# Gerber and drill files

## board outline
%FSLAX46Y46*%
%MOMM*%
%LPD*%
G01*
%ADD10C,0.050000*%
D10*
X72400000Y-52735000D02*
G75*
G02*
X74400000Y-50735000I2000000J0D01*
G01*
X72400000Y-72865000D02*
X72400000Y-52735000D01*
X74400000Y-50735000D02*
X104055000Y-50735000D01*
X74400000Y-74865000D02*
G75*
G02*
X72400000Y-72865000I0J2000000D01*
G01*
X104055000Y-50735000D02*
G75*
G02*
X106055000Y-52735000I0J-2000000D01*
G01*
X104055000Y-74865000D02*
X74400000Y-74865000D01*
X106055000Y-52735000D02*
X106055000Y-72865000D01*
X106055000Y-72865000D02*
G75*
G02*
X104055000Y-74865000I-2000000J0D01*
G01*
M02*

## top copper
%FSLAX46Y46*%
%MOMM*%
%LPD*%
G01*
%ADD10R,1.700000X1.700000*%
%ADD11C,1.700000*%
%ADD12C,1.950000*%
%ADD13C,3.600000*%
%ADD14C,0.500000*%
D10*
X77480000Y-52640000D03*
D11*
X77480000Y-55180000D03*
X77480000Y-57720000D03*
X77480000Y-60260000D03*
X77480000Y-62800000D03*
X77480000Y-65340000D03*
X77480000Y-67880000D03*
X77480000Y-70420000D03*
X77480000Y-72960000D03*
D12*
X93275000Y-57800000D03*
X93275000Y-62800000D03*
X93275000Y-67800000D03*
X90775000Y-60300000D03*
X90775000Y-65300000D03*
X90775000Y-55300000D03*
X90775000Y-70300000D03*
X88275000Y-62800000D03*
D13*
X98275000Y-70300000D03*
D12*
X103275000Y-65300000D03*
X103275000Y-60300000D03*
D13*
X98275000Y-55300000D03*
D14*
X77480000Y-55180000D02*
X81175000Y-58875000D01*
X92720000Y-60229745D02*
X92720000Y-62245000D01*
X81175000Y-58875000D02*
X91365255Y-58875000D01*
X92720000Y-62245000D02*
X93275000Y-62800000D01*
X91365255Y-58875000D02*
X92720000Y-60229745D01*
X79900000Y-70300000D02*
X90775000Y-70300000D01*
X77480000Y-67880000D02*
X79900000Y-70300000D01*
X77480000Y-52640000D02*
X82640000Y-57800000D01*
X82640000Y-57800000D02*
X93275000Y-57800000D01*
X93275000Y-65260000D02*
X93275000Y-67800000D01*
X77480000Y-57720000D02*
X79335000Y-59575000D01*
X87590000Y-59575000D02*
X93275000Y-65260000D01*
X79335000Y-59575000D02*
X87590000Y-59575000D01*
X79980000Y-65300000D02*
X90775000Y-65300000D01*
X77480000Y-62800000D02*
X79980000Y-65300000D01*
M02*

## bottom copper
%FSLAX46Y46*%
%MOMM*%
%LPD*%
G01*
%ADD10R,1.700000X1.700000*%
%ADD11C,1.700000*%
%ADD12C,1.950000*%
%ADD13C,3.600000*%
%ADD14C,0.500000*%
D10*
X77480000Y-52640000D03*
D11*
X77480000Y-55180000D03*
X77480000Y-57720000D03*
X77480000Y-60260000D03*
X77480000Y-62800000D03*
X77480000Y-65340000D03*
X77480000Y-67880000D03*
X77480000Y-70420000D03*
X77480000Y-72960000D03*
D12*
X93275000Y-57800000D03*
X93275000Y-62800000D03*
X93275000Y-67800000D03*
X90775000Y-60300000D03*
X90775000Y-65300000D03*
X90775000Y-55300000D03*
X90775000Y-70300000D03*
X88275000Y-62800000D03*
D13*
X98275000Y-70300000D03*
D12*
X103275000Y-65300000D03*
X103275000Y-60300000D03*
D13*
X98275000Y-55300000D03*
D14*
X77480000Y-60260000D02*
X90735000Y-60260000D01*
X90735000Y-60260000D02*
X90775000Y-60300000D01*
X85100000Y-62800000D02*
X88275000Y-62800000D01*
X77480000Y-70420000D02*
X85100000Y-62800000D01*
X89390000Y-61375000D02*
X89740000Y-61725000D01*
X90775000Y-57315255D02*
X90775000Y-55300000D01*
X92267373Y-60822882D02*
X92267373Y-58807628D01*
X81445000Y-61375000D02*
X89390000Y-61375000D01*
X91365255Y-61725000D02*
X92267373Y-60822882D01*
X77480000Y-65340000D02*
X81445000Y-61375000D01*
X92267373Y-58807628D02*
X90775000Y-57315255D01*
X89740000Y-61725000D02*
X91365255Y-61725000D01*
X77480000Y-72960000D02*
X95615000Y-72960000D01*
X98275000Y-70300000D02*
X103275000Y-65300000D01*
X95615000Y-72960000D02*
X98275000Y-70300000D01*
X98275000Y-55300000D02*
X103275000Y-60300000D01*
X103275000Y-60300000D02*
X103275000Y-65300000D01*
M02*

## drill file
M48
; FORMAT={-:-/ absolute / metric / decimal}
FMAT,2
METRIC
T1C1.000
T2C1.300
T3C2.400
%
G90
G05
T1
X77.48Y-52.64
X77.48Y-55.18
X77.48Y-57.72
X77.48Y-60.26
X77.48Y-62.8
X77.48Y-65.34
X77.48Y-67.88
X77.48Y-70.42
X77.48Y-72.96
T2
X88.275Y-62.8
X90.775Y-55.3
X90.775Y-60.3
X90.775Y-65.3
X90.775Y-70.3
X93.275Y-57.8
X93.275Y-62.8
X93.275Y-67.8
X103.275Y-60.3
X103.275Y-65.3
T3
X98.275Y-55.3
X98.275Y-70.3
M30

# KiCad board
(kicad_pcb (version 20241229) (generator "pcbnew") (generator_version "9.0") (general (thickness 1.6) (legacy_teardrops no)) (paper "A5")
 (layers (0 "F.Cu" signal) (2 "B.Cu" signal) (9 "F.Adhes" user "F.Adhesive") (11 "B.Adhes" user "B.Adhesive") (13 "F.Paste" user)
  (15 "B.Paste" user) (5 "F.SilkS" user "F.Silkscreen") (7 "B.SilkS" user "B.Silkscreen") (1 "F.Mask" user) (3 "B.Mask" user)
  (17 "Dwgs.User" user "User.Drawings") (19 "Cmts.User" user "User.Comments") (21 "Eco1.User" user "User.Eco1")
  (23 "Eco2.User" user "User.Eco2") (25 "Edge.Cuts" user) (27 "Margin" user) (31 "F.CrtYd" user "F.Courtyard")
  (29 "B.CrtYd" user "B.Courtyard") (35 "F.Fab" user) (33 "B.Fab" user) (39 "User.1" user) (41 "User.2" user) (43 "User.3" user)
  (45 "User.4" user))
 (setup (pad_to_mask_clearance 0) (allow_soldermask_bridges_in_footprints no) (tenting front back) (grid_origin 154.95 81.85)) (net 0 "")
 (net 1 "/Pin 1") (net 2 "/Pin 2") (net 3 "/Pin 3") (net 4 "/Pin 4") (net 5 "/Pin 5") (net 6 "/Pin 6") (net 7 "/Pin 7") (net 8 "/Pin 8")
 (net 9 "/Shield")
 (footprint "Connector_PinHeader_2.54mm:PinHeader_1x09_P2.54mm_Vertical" (layer "F.Cu") (at 77.48 52.64)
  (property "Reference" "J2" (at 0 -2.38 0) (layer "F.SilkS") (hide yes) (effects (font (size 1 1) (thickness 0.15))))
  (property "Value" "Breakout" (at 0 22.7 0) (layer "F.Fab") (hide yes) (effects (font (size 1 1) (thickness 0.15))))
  (pad "1" thru_hole rect (at 0 0) (size 1.7 1.7) (drill 1) (layers "*.Cu" "*.Mask") (remove_unused_layers no) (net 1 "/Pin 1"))
  (pad "2" thru_hole circle (at 0 2.54) (size 1.7 1.7) (drill 1) (layers "*.Cu" "*.Mask") (remove_unused_layers no) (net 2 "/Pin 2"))
  (pad "3" thru_hole circle (at 0 5.08) (size 1.7 1.7) (drill 1) (layers "*.Cu" "*.Mask") (remove_unused_layers no) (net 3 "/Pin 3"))
  (pad "4" thru_hole circle (at 0 7.62) (size 1.7 1.7) (drill 1) (layers "*.Cu" "*.Mask") (remove_unused_layers no) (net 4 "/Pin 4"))
  (pad "5" thru_hole circle (at 0 10.16) (size 1.7 1.7) (drill 1) (layers "*.Cu" "*.Mask") (remove_unused_layers no) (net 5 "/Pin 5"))
  (pad "6" thru_hole circle (at 0 12.7) (size 1.7 1.7) (drill 1) (layers "*.Cu" "*.Mask") (remove_unused_layers no) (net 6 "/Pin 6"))
  (pad "7" thru_hole circle (at 0 15.24) (size 1.7 1.7) (drill 1) (layers "*.Cu" "*.Mask") (remove_unused_layers no) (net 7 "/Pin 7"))
  (pad "8" thru_hole circle (at 0 17.78) (size 1.7 1.7) (drill 1) (layers "*.Cu" "*.Mask") (remove_unused_layers no) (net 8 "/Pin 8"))
  (pad "SH" thru_hole circle (at 0 20.32) (size 1.7 1.7) (drill 1) (layers "*.Cu" "*.Mask") (remove_unused_layers no) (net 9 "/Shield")))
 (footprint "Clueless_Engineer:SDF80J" (layer "F.Cu") (at 93.275 57.8 90)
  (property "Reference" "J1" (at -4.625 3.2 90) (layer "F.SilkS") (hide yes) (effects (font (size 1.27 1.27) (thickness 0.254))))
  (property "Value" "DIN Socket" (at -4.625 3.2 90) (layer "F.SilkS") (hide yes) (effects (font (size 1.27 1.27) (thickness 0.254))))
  (pad "1" thru_hole circle (at 0 0 90) (size 1.95 1.95) (drill 1.3) (layers "*.Cu" "*.Mask") (remove_unused_layers no) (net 1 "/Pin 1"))
  (pad "2" thru_hole circle (at -5 0 90) (size 1.95 1.95) (drill 1.3) (layers "*.Cu" "*.Mask") (remove_unused_layers no) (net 2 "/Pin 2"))
  (pad "3" thru_hole circle (at -10 0 90) (size 1.95 1.95) (drill 1.3) (layers "*.Cu" "*.Mask") (remove_unused_layers no) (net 3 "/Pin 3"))
  (pad "4" thru_hole circle (at -2.5 -2.5 90) (size 1.95 1.95) (drill 1.3) (layers "*.Cu" "*.Mask") (remove_unused_layers no)
   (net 4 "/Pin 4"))
  (pad "5" thru_hole circle (at -7.5 -2.5 90) (size 1.95 1.95) (drill 1.3) (layers "*.Cu" "*.Mask") (remove_unused_layers no)
   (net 5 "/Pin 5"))
  (pad "6" thru_hole circle (at 2.5 -2.5 90) (size 1.95 1.95) (drill 1.3) (layers "*.Cu" "*.Mask") (remove_unused_layers no)
   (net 6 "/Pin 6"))
  (pad "7" thru_hole circle (at -12.5 -2.5 90) (size 1.95 1.95) (drill 1.3) (layers "*.Cu" "*.Mask") (remove_unused_layers no)
   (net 7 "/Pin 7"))
  (pad "8" thru_hole circle (at -5 -5 90) (size 1.95 1.95) (drill 1.3) (layers "*.Cu" "*.Mask") (remove_unused_layers no) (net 8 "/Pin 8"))
  (pad "SH" thru_hole circle (at -12.5 5 90) (size 3.6 3.6) (drill 2.4) (layers "*.Cu" "*.Mask") (remove_unused_layers no) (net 9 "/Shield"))
  (pad "SH" thru_hole circle (at -7.5 10 90) (size 1.95 1.95) (drill 1.3) (layers "*.Cu" "*.Mask") (remove_unused_layers no)
   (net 9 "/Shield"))
  (pad "SH" thru_hole circle (at -2.5 10 90) (size 1.95 1.95) (drill 1.3) (layers "*.Cu" "*.Mask") (remove_unused_layers no)
   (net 9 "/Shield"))
  (pad "SH" thru_hole circle (at 2.5 5 90) (size 3.6 3.6) (drill 2.4) (layers "*.Cu" "*.Mask") (remove_unused_layers no) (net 9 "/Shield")))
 (gr_arc (start 72.4 52.735) (mid 72.985786 51.320786) (end 74.4 50.735) (stroke (width 0.05) (type default)) (layer "Edge.Cuts"))
 (gr_line (start 72.4 72.865) (end 72.4 52.735) (stroke (width 0.05) (type default)) (layer "Edge.Cuts"))
 (gr_line (start 74.4 50.735) (end 104.055 50.735) (stroke (width 0.05) (type default)) (layer "Edge.Cuts"))
 (gr_arc (start 74.4 74.865) (mid 72.985786 74.279214) (end 72.4 72.865) (stroke (width 0.05) (type default)) (layer "Edge.Cuts"))
 (gr_arc (start 104.055 50.735) (mid 105.469214 51.320786) (end 106.055 52.735) (stroke (width 0.05) (type default)) (layer "Edge.Cuts"))
 (gr_line (start 104.055 74.865) (end 74.4 74.865) (stroke (width 0.05) (type default)) (layer "Edge.Cuts"))
 (gr_line (start 106.055 52.735) (end 106.055 72.865) (stroke (width 0.05) (type default)) (layer "Edge.Cuts"))
 (gr_arc (start 106.055 72.865) (mid 105.469214 74.279214) (end 104.055 74.865) (stroke (width 0.05) (type default)) (layer "Edge.Cuts"))
 (segment (start 77.48 60.26) (end 90.735 60.26) (width 0.5) (layer "B.Cu") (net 4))
 (segment (start 90.735 60.26) (end 90.775 60.3) (width 0.5) (layer "B.Cu") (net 4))
 (segment (start 85.1 62.8) (end 88.275 62.8) (width 0.5) (layer "B.Cu") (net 8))
 (segment (start 77.48 70.42) (end 85.1 62.8) (width 0.5) (layer "B.Cu") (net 8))
 (segment (start 77.48 55.18) (end 81.175 58.875) (width 0.5) (layer "F.Cu") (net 2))
 (segment (start 92.72 60.229745) (end 92.72 62.245) (width 0.5) (layer "F.Cu") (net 2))
 (segment (start 81.175 58.875) (end 91.365255 58.875) (width 0.5) (layer "F.Cu") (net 2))
 (segment (start 92.72 62.245) (end 93.275 62.8) (width 0.5) (layer "F.Cu") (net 2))
 (segment (start 91.365255 58.875) (end 92.72 60.229745) (width 0.5) (layer "F.Cu") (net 2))
 (segment (start 89.39 61.375) (end 89.74 61.725) (width 0.5) (layer "B.Cu") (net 6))
 (segment (start 90.775 57.315255) (end 90.775 55.3) (width 0.5) (layer "B.Cu") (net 6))
 (segment (start 92.267373 60.822882) (end 92.267373 58.807628) (width 0.5) (layer "B.Cu") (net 6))
 (segment (start 81.445 61.375) (end 89.39 61.375) (width 0.5) (layer "B.Cu") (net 6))
 (segment (start 91.365255 61.725) (end 92.267373 60.822882) (width 0.5) (layer "B.Cu") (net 6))
 (segment (start 77.48 65.34) (end 81.445 61.375) (width 0.5) (layer "B.Cu") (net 6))
 (segment (start 92.267373 58.807628) (end 90.775 57.315255) (width 0.5) (layer "B.Cu") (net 6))
 (segment (start 89.74 61.725) (end 91.365255 61.725) (width 0.5) (layer "B.Cu") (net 6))
 (segment (start 79.9 70.3) (end 90.775 70.3) (width 0.5) (layer "F.Cu") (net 7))
 (segment (start 77.48 67.88) (end 79.9 70.3) (width 0.5) (layer "F.Cu") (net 7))
 (segment (start 77.48 52.64) (end 82.64 57.8) (width 0.5) (layer "F.Cu") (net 1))
 (segment (start 82.64 57.8) (end 93.275 57.8) (width 0.5) (layer "F.Cu") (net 1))
 (segment (start 93.275 65.26) (end 93.275 67.8) (width 0.5) (layer "F.Cu") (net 3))
 (segment (start 77.48 57.72) (end 79.335 59.575) (width 0.5) (layer "F.Cu") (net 3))
 (segment (start 87.59 59.575) (end 93.275 65.26) (width 0.5) (layer "F.Cu") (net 3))
 (segment (start 79.335 59.575) (end 87.59 59.575) (width 0.5) (layer "F.Cu") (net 3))
 (segment (start 79.98 65.3) (end 90.775 65.3) (width 0.5) (layer "F.Cu") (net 5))
 (segment (start 77.48 62.8) (end 79.98 65.3) (width 0.5) (layer "F.Cu") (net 5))
 (segment (start 77.48 72.96) (end 95.615 72.96) (width 0.5) (layer "B.Cu") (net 9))
 (segment (start 98.275 70.3) (end 103.275 65.3) (width 0.5) (layer "B.Cu") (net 9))
 (segment (start 95.615 72.96) (end 98.275 70.3) (width 0.5) (layer "B.Cu") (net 9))
 (segment (start 98.275 55.3) (end 103.275 60.3) (width 0.5) (layer "B.Cu") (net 9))
 (segment (start 103.275 60.3) (end 103.275 65.3) (width 0.5) (layer "B.Cu") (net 9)))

